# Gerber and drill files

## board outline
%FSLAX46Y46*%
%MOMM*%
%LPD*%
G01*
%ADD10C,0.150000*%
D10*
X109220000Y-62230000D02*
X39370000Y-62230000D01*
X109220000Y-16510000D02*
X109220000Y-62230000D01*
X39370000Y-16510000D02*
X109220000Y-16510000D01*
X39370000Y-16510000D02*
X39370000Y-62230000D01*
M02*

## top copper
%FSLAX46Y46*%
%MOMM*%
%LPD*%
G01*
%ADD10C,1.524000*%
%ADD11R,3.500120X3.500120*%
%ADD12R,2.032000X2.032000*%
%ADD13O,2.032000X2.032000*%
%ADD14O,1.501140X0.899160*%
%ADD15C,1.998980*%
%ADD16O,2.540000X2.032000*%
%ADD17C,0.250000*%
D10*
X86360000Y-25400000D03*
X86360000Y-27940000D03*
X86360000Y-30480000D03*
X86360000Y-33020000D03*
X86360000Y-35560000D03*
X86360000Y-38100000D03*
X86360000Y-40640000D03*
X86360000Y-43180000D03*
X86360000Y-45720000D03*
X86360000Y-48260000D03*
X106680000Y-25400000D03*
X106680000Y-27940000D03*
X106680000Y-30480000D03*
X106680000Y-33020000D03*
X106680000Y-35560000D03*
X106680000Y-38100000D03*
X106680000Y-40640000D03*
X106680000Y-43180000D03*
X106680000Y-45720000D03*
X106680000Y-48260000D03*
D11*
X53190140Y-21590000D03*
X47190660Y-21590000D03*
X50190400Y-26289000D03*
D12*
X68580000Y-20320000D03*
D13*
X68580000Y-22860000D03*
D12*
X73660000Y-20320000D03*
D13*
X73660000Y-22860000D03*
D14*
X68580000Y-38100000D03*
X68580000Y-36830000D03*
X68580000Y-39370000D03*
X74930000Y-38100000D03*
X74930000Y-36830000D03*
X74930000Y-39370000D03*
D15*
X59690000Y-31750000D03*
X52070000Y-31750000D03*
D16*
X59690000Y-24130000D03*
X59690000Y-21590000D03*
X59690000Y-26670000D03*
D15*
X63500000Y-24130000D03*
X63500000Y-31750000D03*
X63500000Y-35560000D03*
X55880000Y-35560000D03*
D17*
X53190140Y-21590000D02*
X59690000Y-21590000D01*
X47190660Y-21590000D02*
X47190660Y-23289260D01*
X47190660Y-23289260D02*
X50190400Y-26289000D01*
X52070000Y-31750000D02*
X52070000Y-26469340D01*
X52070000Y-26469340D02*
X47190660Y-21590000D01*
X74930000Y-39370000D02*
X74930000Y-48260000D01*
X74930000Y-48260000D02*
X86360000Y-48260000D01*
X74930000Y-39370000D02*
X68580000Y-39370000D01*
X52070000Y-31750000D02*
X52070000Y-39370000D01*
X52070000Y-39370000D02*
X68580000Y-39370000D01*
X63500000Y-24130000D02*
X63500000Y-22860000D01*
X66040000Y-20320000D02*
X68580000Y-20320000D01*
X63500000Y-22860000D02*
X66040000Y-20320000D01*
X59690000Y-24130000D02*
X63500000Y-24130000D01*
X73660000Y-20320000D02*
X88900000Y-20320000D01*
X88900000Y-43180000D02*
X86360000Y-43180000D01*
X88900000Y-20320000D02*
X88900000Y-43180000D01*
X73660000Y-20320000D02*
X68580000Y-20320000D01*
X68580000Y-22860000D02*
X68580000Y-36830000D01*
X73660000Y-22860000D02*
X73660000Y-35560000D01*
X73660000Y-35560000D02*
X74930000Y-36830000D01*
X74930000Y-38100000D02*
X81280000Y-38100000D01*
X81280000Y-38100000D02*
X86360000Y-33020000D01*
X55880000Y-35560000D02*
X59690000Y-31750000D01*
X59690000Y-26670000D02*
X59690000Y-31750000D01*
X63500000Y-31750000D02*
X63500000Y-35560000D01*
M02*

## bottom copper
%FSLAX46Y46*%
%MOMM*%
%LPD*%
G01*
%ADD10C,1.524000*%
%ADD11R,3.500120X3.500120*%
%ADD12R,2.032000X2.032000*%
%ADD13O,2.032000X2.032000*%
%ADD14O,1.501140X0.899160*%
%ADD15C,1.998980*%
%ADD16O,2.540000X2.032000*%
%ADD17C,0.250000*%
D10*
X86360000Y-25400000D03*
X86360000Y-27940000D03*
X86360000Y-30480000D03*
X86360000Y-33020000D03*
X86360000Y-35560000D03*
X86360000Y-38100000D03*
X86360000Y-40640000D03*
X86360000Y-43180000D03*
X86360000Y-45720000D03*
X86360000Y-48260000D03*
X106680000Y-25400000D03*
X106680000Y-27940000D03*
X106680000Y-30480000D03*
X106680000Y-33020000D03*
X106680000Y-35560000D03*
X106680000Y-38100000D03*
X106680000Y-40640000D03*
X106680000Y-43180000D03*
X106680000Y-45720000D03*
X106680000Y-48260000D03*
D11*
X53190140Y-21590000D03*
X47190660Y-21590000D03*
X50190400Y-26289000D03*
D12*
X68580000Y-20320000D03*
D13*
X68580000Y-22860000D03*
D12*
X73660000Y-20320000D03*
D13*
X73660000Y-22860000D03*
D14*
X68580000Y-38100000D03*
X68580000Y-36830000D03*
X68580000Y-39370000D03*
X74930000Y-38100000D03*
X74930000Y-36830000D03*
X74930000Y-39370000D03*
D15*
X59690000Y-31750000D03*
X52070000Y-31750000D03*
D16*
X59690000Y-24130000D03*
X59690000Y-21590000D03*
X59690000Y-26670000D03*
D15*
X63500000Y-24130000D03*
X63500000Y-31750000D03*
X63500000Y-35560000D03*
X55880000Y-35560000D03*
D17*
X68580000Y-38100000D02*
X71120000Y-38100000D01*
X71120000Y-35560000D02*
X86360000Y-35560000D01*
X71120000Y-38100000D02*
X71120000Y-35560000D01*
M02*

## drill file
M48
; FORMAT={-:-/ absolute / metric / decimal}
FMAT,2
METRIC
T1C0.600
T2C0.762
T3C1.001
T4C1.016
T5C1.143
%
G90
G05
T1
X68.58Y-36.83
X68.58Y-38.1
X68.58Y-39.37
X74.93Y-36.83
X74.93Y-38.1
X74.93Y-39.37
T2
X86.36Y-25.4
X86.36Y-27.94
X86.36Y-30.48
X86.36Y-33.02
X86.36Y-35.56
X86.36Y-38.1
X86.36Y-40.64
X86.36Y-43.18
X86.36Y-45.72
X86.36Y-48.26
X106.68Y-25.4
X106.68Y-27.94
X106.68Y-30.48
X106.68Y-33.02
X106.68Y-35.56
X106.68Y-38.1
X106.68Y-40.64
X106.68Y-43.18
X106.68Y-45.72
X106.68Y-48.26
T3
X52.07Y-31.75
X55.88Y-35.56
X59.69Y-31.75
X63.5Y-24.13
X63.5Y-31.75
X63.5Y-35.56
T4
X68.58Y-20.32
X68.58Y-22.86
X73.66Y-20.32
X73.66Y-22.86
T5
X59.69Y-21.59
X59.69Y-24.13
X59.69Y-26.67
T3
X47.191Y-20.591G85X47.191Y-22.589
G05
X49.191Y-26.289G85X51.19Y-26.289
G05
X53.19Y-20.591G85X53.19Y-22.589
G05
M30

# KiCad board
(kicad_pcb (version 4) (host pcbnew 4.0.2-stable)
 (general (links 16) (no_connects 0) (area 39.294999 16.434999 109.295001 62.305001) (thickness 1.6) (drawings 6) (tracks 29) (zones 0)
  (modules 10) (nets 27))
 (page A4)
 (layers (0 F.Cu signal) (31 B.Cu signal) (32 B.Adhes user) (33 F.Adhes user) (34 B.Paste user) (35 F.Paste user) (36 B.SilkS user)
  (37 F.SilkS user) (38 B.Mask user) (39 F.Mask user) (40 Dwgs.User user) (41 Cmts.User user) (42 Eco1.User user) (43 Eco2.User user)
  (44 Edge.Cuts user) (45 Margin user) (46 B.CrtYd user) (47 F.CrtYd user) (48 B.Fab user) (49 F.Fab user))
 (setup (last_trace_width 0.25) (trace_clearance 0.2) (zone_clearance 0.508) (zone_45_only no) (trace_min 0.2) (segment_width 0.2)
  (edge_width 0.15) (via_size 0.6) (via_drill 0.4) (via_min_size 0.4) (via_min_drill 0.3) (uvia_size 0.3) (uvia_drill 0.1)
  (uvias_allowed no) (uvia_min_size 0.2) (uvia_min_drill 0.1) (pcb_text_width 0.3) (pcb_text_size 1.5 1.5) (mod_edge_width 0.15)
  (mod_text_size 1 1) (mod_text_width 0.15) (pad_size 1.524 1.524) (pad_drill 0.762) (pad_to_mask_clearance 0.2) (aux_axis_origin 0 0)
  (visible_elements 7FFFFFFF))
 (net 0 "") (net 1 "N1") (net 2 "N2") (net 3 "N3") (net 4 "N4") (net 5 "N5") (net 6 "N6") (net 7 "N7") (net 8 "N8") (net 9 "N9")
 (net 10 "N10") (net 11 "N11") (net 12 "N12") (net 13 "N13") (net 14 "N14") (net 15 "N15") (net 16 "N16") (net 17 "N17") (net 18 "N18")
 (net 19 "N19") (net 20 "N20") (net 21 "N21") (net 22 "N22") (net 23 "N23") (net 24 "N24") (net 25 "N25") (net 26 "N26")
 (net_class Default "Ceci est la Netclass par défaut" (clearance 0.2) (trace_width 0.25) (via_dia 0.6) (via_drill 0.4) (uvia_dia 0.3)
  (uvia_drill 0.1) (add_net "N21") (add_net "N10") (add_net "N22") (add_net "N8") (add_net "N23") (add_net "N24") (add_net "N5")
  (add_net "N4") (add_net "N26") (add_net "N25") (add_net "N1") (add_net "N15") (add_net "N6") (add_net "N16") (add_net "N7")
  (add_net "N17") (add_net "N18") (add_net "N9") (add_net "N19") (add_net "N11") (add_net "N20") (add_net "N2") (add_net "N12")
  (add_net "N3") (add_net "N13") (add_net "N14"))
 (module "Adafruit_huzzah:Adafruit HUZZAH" (layer F.Cu) (at 83.82 20.32)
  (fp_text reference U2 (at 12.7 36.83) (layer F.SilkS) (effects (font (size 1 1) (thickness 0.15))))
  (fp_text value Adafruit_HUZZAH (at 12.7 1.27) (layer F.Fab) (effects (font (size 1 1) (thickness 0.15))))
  (pad 1 thru_hole circle (at 2.54 5.08) (size 1.524 1.524) (drill 0.762) (layers *.Cu *.Mask F.SilkS) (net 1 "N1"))
  (pad 3 thru_hole circle (at 2.54 7.62) (size 1.524 1.524) (drill 0.762) (layers *.Cu *.Mask F.SilkS) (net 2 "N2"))
  (pad 5 thru_hole circle (at 2.54 10.16) (size 1.524 1.524) (drill 0.762) (layers *.Cu *.Mask F.SilkS) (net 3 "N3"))
  (pad 7 thru_hole circle (at 2.54 12.7) (size 1.524 1.524) (drill 0.762) (layers *.Cu *.Mask F.SilkS) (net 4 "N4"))
  (pad 9 thru_hole circle (at 2.54 15.24) (size 1.524 1.524) (drill 0.762) (layers *.Cu *.Mask F.SilkS) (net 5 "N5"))
  (pad 11 thru_hole circle (at 2.54 17.78) (size 1.524 1.524) (drill 0.762) (layers *.Cu *.Mask F.SilkS) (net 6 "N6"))
  (pad 13 thru_hole circle (at 2.54 20.32) (size 1.524 1.524) (drill 0.762) (layers *.Cu *.Mask F.SilkS) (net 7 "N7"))
  (pad 15 thru_hole circle (at 2.54 22.86) (size 1.524 1.524) (drill 0.762) (layers *.Cu *.Mask F.SilkS) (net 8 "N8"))
  (pad 17 thru_hole circle (at 2.54 25.4) (size 1.524 1.524) (drill 0.762) (layers *.Cu *.Mask F.SilkS) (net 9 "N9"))
  (pad 19 thru_hole circle (at 2.54 27.94) (size 1.524 1.524) (drill 0.762) (layers *.Cu *.Mask F.SilkS) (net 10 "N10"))
  (pad 2 thru_hole circle (at 22.86 5.08) (size 1.524 1.524) (drill 0.762) (layers *.Cu *.Mask F.SilkS) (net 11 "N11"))
  (pad 4 thru_hole circle (at 22.86 7.62) (size 1.524 1.524) (drill 0.762) (layers *.Cu *.Mask F.SilkS) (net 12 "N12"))
  (pad 6 thru_hole circle (at 22.86 10.16) (size 1.524 1.524) (drill 0.762) (layers *.Cu *.Mask F.SilkS) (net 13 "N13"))
  (pad 8 thru_hole circle (at 22.86 12.7) (size 1.524 1.524) (drill 0.762) (layers *.Cu *.Mask F.SilkS) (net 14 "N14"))
  (pad 10 thru_hole circle (at 22.86 15.24) (size 1.524 1.524) (drill 0.762) (layers *.Cu *.Mask F.SilkS) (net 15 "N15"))
  (pad 12 thru_hole circle (at 22.86 17.78) (size 1.524 1.524) (drill 0.762) (layers *.Cu *.Mask F.SilkS) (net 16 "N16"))
  (pad 14 thru_hole circle (at 22.86 20.32) (size 1.524 1.524) (drill 0.762) (layers *.Cu *.Mask F.SilkS) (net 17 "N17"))
  (pad 16 thru_hole circle (at 22.86 22.86) (size 1.524 1.524) (drill 0.762) (layers *.Cu *.Mask F.SilkS) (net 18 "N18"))
  (pad 18 thru_hole circle (at 22.86 25.4) (size 1.524 1.524) (drill 0.762) (layers *.Cu *.Mask F.SilkS) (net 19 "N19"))
  (pad 20 thru_hole circle (at 22.86 27.94) (size 1.524 1.524) (drill 0.762) (layers *.Cu *.Mask F.SilkS) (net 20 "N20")))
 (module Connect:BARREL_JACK (layer F.Cu) (at 46.99 21.59)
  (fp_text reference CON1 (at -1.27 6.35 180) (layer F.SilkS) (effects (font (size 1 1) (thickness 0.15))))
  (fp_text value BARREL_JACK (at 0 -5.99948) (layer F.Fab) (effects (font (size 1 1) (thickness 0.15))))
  (pad 1 thru_hole rect (at 6.20014 0) (size 3.50012 3.50012) (drill oval 1.00076 2.99974) (layers *.Cu *.Mask F.SilkS) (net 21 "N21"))
  (pad 2 thru_hole rect (at 0.20066 0) (size 3.50012 3.50012) (drill oval 1.00076 2.99974) (layers *.Cu *.Mask F.SilkS) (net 10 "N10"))
  (pad 3 thru_hole rect (at 3.2004 4.699) (size 3.50012 3.50012) (drill oval 2.99974 1.00076) (layers *.Cu *.Mask F.SilkS) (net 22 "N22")))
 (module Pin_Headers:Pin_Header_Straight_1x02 (layer F.Cu) (at 68.58 20.32)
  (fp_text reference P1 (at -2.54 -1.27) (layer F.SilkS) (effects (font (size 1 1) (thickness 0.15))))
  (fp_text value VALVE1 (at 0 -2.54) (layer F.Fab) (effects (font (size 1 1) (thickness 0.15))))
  (pad 1 thru_hole rect (at 0 0) (size 2.032 2.032) (drill 1.016) (layers *.Cu *.Mask F.SilkS) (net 8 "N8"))
  (pad 2 thru_hole oval (at 0 2.54) (size 2.032 2.032) (drill 1.016) (layers *.Cu *.Mask F.SilkS) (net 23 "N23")))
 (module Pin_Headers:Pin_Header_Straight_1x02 (layer F.Cu) (at 73.66 20.32)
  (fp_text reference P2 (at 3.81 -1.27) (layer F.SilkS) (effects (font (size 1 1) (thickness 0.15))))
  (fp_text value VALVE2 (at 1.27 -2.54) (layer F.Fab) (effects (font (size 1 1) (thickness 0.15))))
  (pad 1 thru_hole rect (at 0 0) (size 2.032 2.032) (drill 1.016) (layers *.Cu *.Mask F.SilkS) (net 8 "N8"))
  (pad 2 thru_hole oval (at 0 2.54) (size 2.032 2.032) (drill 1.016) (layers *.Cu *.Mask F.SilkS) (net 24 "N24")))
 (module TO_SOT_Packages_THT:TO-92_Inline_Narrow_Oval (layer F.Cu) (at 68.58 39.37 90)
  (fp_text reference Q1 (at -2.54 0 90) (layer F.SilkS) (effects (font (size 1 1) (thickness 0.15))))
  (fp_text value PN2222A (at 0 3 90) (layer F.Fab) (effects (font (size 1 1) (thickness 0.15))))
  (pad 2 thru_hole oval (at 1.27 0 270) (size 0.89916 1.50114) (drill 0.6) (layers *.Cu *.Mask F.SilkS) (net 5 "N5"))
  (pad 3 thru_hole oval (at 2.54 0 270) (size 0.89916 1.50114) (drill 0.6) (layers *.Cu *.Mask F.SilkS) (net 23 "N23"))
  (pad 1 thru_hole oval (at 0 0 270) (size 0.89916 1.50114) (drill 0.6) (layers *.Cu *.Mask F.SilkS) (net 10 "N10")))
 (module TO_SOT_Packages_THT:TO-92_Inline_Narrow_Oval (layer F.Cu) (at 74.93 39.37 90)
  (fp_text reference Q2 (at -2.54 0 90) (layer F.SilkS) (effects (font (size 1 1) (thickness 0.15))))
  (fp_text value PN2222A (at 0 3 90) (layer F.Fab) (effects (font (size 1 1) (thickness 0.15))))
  (pad 2 thru_hole oval (at 1.27 0 270) (size 0.89916 1.50114) (drill 0.6) (layers *.Cu *.Mask F.SilkS) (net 4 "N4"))
  (pad 3 thru_hole oval (at 2.54 0 270) (size 0.89916 1.50114) (drill 0.6) (layers *.Cu *.Mask F.SilkS) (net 24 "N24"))
  (pad 1 thru_hole oval (at 0 0 270) (size 0.89916 1.50114) (drill 0.6) (layers *.Cu *.Mask F.SilkS) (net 10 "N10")))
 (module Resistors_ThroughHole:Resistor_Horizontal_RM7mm (layer F.Cu) (at 59.69 31.75 180)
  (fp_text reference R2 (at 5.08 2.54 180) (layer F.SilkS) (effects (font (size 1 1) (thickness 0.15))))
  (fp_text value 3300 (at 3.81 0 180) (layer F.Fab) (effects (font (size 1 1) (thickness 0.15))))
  (pad 1 thru_hole circle (at 0 0 180) (size 1.99898 1.99898) (drill 1.00076) (layers *.Cu *.SilkS *.Mask) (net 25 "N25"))
  (pad 2 thru_hole circle (at 7.62 0 180) (size 1.99898 1.99898) (drill 1.00076) (layers *.Cu *.SilkS *.Mask) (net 10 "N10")))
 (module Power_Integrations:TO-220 (layer F.Cu) (at 59.69 24.13 90)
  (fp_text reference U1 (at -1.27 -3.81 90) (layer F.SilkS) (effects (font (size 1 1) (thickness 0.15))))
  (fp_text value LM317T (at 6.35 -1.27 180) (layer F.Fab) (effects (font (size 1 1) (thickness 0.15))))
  (pad 2 thru_hole oval (at 0 0 90) (size 2.032 2.54) (drill 1.143) (layers *.Cu *.Mask F.SilkS) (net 8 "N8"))
  (pad 3 thru_hole oval (at 2.54 0 90) (size 2.032 2.54) (drill 1.143) (layers *.Cu *.Mask F.SilkS) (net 21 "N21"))
  (pad 1 thru_hole oval (at -2.54 0 90) (size 2.032 2.54) (drill 1.143) (layers *.Cu *.Mask F.SilkS) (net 25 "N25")))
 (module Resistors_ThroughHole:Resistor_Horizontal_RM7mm (layer F.Cu) (at 63.5 24.13 270)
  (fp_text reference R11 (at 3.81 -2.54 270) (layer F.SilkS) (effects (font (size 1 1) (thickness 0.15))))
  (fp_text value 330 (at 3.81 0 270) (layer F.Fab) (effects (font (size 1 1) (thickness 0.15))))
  (pad 1 thru_hole circle (at 0 0 270) (size 1.99898 1.99898) (drill 1.00076) (layers *.Cu *.SilkS *.Mask) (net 8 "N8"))
  (pad 2 thru_hole circle (at 7.62 0 270) (size 1.99898 1.99898) (drill 1.00076) (layers *.Cu *.SilkS *.Mask) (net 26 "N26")))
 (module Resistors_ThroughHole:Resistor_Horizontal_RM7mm (layer F.Cu) (at 63.5 35.56 180)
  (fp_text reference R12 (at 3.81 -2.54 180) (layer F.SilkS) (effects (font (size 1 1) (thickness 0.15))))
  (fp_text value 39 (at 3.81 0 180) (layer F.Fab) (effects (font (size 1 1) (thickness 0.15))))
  (pad 1 thru_hole circle (at 0 0 180) (size 1.99898 1.99898) (drill 1.00076) (layers *.Cu *.SilkS *.Mask) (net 26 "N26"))
  (pad 2 thru_hole circle (at 7.62 0 180) (size 1.99898 1.99898) (drill 1.00076) (layers *.Cu *.SilkS *.Mask) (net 25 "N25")))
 (gr_line (start 109.22 62.23) (end 39.37 62.23) (angle 90) (layer Edge.Cuts) (width 0.15))
 (gr_line (start 109.22 16.51) (end 109.22 62.23) (angle 90) (layer Edge.Cuts) (width 0.15))
 (gr_line (start 39.37 16.51) (end 109.22 16.51) (angle 90) (layer Edge.Cuts) (width 0.15))
 (gr_line (start 39.37 16.51) (end 39.37 62.23) (angle 90) (layer Edge.Cuts) (width 0.15))
 (segment (start 53.19014 21.59) (end 59.69 21.59) (width 0.25) (layer F.Cu) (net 21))
 (segment (start 47.19066 21.59) (end 47.19066 23.28926) (width 0.25) (layer F.Cu) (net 10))
 (segment (start 47.19066 23.28926) (end 50.1904 26.289) (width 0.25) (layer F.Cu) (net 10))
 (segment (start 52.07 31.75) (end 52.07 26.46934) (width 0.25) (layer F.Cu) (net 10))
 (segment (start 52.07 26.46934) (end 47.19066 21.59) (width 0.25) (layer F.Cu) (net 10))
 (segment (start 74.93 39.37) (end 74.93 48.26) (width 0.25) (layer F.Cu) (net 10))
 (segment (start 74.93 48.26) (end 86.36 48.26) (width 0.25) (layer F.Cu) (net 10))
 (segment (start 74.93 39.37) (end 68.58 39.37) (width 0.25) (layer F.Cu) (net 10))
 (segment (start 52.07 31.75) (end 52.07 39.37) (width 0.25) (layer F.Cu) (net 10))
 (segment (start 52.07 39.37) (end 68.58 39.37) (width 0.25) (layer F.Cu) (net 10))
 (segment (start 63.5 24.13) (end 63.5 22.86) (width 0.25) (layer F.Cu) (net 8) (status 400000))
 (segment (start 66.04 20.32) (end 68.58 20.32) (width 0.25) (layer F.Cu) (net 8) (status 800000))
 (segment (start 63.5 22.86) (end 66.04 20.32) (width 0.25) (layer F.Cu) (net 8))
 (segment (start 59.69 24.13) (end 63.5 24.13) (width 0.25) (layer F.Cu) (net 8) (status C00000))
 (segment (start 73.66 20.32) (end 88.9 20.32) (width 0.25) (layer F.Cu) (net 8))
 (segment (start 88.9 43.18) (end 86.36 43.18) (width 0.25) (layer F.Cu) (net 8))
 (segment (start 88.9 20.32) (end 88.9 43.18) (width 0.25) (layer F.Cu) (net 8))
 (segment (start 73.66 20.32) (end 68.58 20.32) (width 0.25) (layer F.Cu) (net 8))
 (segment (start 68.58 22.86) (end 68.58 36.83) (width 0.25) (layer F.Cu) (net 23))
 (segment (start 73.66 22.86) (end 73.66 35.56) (width 0.25) (layer F.Cu) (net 24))
 (segment (start 73.66 35.56) (end 74.93 36.83) (width 0.25) (layer F.Cu) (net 24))
 (segment (start 68.58 38.1) (end 71.12 38.1) (width 0.25) (layer B.Cu) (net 5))
 (segment (start 71.12 35.56) (end 86.36 35.56) (width 0.25) (layer B.Cu) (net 5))
 (segment (start 71.12 38.1) (end 71.12 35.56) (width 0.25) (layer B.Cu) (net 5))
 (segment (start 74.93 38.1) (end 81.28 38.1) (width 0.25) (layer F.Cu) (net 4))
 (segment (start 81.28 38.1) (end 86.36 33.02) (width 0.25) (layer F.Cu) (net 4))
 (segment (start 55.88 35.56) (end 59.69 31.75) (width 0.25) (layer F.Cu) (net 25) (status C00000))
 (segment (start 59.69 26.67) (end 59.69 31.75) (width 0.25) (layer F.Cu) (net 25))
 (segment (start 63.5 31.75) (end 63.5 35.56) (width 0.25) (layer F.Cu) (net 26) (status C00000)))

